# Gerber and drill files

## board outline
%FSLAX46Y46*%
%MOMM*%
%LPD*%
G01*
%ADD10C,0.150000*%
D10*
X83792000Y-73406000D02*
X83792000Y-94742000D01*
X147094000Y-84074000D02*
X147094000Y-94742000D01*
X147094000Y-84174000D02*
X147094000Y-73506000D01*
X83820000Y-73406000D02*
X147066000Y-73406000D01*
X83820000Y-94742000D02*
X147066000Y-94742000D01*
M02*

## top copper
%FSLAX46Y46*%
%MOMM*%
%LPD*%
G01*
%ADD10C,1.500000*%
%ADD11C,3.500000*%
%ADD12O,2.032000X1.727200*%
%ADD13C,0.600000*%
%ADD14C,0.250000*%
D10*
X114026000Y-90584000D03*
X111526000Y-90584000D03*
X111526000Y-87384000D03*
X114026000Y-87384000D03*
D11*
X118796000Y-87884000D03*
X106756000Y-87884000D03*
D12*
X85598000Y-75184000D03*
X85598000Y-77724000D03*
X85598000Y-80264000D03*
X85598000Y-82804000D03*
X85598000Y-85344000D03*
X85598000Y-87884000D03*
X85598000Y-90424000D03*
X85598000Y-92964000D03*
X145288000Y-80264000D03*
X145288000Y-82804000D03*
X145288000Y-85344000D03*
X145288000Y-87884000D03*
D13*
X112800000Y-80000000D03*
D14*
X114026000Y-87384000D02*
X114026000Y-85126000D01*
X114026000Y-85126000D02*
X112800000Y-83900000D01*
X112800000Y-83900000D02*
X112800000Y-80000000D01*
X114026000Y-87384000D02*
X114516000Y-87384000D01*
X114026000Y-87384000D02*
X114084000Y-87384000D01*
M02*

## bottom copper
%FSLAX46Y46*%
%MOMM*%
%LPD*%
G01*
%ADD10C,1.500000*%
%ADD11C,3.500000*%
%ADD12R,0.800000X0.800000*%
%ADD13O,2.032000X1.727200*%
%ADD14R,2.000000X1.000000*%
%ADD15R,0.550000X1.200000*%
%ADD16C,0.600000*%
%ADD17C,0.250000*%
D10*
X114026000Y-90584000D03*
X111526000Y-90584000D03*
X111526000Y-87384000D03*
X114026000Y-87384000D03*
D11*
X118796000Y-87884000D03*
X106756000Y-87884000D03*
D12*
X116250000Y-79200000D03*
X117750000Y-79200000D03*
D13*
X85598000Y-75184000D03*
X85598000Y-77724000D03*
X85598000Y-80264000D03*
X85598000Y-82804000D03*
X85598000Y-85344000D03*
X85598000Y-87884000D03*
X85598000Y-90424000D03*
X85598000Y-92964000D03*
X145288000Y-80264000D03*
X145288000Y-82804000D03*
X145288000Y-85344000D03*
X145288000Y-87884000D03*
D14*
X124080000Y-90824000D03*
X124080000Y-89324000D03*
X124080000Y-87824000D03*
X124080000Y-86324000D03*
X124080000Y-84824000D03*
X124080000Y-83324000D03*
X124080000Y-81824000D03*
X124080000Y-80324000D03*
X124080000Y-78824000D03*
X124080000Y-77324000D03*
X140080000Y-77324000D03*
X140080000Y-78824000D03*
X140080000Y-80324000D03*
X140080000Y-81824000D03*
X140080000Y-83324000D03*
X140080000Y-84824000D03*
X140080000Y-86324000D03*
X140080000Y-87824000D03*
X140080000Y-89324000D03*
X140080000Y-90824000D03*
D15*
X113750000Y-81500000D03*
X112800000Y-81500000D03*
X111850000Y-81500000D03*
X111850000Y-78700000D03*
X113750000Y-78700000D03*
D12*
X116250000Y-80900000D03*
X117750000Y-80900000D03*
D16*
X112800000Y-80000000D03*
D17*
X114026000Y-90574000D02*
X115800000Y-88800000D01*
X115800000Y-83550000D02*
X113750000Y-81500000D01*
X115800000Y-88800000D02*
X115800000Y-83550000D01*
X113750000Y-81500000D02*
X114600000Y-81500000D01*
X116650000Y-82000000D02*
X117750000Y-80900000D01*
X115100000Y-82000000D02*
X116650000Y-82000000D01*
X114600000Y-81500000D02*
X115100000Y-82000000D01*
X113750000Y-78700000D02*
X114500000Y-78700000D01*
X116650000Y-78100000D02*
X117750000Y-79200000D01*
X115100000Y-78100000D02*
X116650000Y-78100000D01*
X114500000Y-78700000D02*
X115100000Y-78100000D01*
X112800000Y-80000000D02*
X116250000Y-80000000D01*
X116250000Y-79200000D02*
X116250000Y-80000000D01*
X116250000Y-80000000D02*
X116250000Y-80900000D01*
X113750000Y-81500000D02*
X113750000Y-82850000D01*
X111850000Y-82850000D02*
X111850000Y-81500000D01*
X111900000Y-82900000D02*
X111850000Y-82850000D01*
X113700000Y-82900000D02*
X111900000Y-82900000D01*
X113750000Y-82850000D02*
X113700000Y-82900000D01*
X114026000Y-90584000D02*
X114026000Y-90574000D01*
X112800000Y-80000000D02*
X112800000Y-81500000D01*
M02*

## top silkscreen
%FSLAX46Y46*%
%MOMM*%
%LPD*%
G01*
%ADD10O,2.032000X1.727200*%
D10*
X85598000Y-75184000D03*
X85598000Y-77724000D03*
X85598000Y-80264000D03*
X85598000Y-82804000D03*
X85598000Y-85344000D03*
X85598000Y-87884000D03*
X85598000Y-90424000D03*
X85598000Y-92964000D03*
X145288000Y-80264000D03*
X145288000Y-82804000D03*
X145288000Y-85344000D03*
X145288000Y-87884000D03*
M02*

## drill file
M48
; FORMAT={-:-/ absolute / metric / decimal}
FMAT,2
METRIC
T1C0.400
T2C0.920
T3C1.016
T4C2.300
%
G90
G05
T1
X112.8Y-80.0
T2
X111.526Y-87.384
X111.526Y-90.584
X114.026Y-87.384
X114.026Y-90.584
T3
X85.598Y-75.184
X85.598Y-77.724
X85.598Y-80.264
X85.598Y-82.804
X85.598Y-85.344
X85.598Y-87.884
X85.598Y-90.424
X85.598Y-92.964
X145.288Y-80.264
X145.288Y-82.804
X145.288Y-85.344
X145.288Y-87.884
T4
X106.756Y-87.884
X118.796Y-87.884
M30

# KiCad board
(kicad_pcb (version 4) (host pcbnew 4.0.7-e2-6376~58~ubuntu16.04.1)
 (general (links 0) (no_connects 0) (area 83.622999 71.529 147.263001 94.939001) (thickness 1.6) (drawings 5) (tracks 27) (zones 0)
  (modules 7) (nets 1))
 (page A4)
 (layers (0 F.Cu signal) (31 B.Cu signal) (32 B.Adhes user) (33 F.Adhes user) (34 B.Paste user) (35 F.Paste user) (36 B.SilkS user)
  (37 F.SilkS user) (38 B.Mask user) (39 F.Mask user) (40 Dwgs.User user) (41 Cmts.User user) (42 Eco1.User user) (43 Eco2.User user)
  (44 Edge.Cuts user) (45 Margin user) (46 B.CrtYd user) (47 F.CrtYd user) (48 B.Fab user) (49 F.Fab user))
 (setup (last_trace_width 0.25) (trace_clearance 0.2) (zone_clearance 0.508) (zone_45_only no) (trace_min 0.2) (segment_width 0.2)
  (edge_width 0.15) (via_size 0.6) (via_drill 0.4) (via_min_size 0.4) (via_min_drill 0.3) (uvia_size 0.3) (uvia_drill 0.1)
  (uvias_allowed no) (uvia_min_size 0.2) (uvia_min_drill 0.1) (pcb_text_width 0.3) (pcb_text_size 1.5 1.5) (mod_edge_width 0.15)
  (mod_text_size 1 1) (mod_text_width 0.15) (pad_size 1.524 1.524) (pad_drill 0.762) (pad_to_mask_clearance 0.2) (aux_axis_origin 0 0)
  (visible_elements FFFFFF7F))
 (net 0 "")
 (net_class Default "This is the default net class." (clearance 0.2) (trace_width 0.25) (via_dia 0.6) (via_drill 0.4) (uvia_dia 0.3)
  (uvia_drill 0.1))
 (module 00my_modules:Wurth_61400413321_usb (layer B.Cu) (at 112.776 87.884)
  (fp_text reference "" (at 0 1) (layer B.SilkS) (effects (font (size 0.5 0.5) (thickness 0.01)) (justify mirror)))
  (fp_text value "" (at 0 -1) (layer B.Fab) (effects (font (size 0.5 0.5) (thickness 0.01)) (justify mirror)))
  (pad V thru_hole circle (at 1.25 2.7) (size 1.5 1.5) (drill 0.92) (layers *.Cu *.Mask B.SilkS))
  (pad - thru_hole circle (at -1.25 2.7) (size 1.5 1.5) (drill 0.92) (layers *.Cu *.Mask B.SilkS))
  (pad + thru_hole circle (at -1.25 -0.5) (size 1.5 1.5) (drill 0.92) (layers *.Cu *.Mask B.SilkS))
  (pad G thru_hole circle (at 1.25 -0.5) (size 1.5 1.5) (drill 0.92) (layers *.Cu *.Mask B.SilkS))
  (pad X thru_hole circle (at 6.02 0) (size 3.5 3.5) (drill 2.3) (layers *.Cu *.Mask B.SilkS))
  (pad X thru_hole circle (at -6.02 0) (size 3.5 3.5) (drill 2.3) (layers *.Cu *.Mask B.SilkS)))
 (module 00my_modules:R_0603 (layer B.Cu) (at 117 79.2)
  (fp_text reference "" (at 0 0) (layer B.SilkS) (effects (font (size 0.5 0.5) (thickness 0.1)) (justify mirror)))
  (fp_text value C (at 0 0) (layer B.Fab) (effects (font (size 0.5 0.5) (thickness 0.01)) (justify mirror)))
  (pad 1 smd rect (at -0.75 0) (size 0.8 0.8) (layers B.Cu B.Paste B.Mask))
  (pad 2 smd rect (at 0.75 0) (size 0.8 0.8) (layers B.Cu B.Paste B.Mask)))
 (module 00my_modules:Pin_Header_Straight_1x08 (layer F.Cu) (at 85.598 75.184)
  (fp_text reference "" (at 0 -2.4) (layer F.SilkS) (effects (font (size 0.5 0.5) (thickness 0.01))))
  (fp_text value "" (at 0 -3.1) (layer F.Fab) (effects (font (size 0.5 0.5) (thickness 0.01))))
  (pad 1 thru_hole oval (at 0 0) (size 2.032 1.7272) (drill 1.016) (layers *.Cu *.Mask F.SilkS))
  (pad 2 thru_hole oval (at 0 2.54) (size 2.032 1.7272) (drill 1.016) (layers *.Cu *.Mask F.SilkS))
  (pad 3 thru_hole oval (at 0 5.08) (size 2.032 1.7272) (drill 1.016) (layers *.Cu *.Mask F.SilkS))
  (pad 4 thru_hole oval (at 0 7.62) (size 2.032 1.7272) (drill 1.016) (layers *.Cu *.Mask F.SilkS))
  (pad 5 thru_hole oval (at 0 10.16) (size 2.032 1.7272) (drill 1.016) (layers *.Cu *.Mask F.SilkS))
  (pad 6 thru_hole oval (at 0 12.7) (size 2.032 1.7272) (drill 1.016) (layers *.Cu *.Mask F.SilkS))
  (pad 7 thru_hole oval (at 0 15.24) (size 2.032 1.7272) (drill 1.016) (layers *.Cu *.Mask F.SilkS))
  (pad 8 thru_hole oval (at 0 17.78) (size 2.032 1.7272) (drill 1.016) (layers *.Cu *.Mask F.SilkS)))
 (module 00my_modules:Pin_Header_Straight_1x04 (layer F.Cu) (at 145.288 80.264)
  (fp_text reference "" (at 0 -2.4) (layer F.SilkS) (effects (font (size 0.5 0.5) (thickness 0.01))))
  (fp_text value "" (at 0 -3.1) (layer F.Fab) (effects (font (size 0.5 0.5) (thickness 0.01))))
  (pad 1 thru_hole oval (at 0 0) (size 2.032 1.7272) (drill 1.016) (layers *.Cu *.Mask F.SilkS))
  (pad 2 thru_hole oval (at 0 2.54) (size 2.032 1.7272) (drill 1.016) (layers *.Cu *.Mask F.SilkS))
  (pad 3 thru_hole oval (at 0 5.08) (size 2.032 1.7272) (drill 1.016) (layers *.Cu *.Mask F.SilkS))
  (pad 4 thru_hole oval (at 0 7.62) (size 2.032 1.7272) (drill 1.016) (layers *.Cu *.Mask F.SilkS)))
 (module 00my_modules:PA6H (layer B.Cu) (at 132.08 84.074)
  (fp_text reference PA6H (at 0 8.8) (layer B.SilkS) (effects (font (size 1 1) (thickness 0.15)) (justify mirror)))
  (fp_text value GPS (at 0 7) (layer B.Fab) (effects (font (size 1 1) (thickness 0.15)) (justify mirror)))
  (pad VCC smd rect (at -8 6.75) (size 2 1) (layers B.Cu B.Paste B.Mask))
  (pad 2 smd rect (at -8 5.25) (size 2 1) (layers B.Cu B.Paste B.Mask))
  (pad GND smd rect (at -8 3.75) (size 2 1) (layers B.Cu B.Paste B.Mask))
  (pad 4 smd rect (at -8 2.25) (size 2 1) (layers B.Cu B.Paste B.Mask))
  (pad 5 smd rect (at -8 0.75) (size 2 1) (layers B.Cu B.Paste B.Mask))
  (pad 6 smd rect (at -8 -0.75) (size 2 1) (layers B.Cu B.Paste B.Mask))
  (pad 7 smd rect (at -8 -2.25) (size 2 1) (layers B.Cu B.Paste B.Mask))
  (pad 8 smd rect (at -8 -3.75) (size 2 1) (layers B.Cu B.Paste B.Mask))
  (pad TX smd rect (at -8 -5.25) (size 2 1) (layers B.Cu B.Paste B.Mask))
  (pad RX smd rect (at -8 -6.75) (size 2 1) (layers B.Cu B.Paste B.Mask))
  (pad 11 smd rect (at 8 -6.75) (size 2 1) (layers B.Cu B.Paste B.Mask))
  (pad 12 smd rect (at 8 -5.25) (size 2 1) (layers B.Cu B.Paste B.Mask))
  (pad 13 smd rect (at 8 -3.75) (size 2 1) (layers B.Cu B.Paste B.Mask))
  (pad 14 smd rect (at 8 -2.25) (size 2 1) (layers B.Cu B.Paste B.Mask))
  (pad 15 smd rect (at 8 -0.75) (size 2 1) (layers B.Cu B.Paste B.Mask))
  (pad 16 smd rect (at 8 0.75) (size 2 1) (layers B.Cu B.Paste B.Mask))
  (pad 17 smd rect (at 8 2.25) (size 2 1) (layers B.Cu B.Paste B.Mask))
  (pad 18 smd rect (at 8 3.75) (size 2 1) (layers B.Cu B.Paste B.Mask))
  (pad 19 smd rect (at 8 5.25) (size 2 1) (layers B.Cu B.Paste B.Mask))
  (pad 20 smd rect (at 8 6.75) (size 2 1) (layers B.Cu B.Paste B.Mask)))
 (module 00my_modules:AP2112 (layer B.Cu) (at 112.8 80.1 90)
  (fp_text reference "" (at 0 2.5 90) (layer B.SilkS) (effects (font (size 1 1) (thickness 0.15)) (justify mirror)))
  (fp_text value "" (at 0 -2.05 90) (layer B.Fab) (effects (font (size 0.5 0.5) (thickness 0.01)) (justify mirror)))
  (pad VIN smd rect (at -1.4 0.95 90) (size 1.2 0.55) (layers B.Cu B.Paste B.Mask))
  (pad GND smd rect (at -1.4 0 90) (size 1.2 0.55) (layers B.Cu B.Paste B.Mask))
  (pad EN smd rect (at -1.4 -0.95 90) (size 1.2 0.55) (layers B.Cu B.Paste B.Mask))
  (pad NC smd rect (at 1.4 -0.95 90) (size 1.2 0.55) (layers B.Cu B.Paste B.Mask))
  (pad VOUT smd rect (at 1.4 0.95 90) (size 1.2 0.55) (layers B.Cu B.Paste B.Mask)))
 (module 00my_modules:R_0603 (layer B.Cu) (at 117 80.9)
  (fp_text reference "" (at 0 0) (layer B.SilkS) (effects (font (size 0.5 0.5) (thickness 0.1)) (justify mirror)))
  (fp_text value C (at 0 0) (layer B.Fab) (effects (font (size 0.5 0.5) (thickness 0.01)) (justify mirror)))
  (pad 1 smd rect (at -0.75 0) (size 0.8 0.8) (layers B.Cu B.Paste B.Mask))
  (pad 2 smd rect (at 0.75 0) (size 0.8 0.8) (layers B.Cu B.Paste B.Mask)))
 (gr_line (start 83.792 73.406) (end 83.792 94.742) (angle 90) (layer Edge.Cuts) (width 0.15))
 (gr_line (start 147.094 84.074) (end 147.094 94.742) (angle 90) (layer Edge.Cuts) (width 0.15))
 (gr_line (start 147.094 84.174) (end 147.094 73.506) (angle 90) (layer Edge.Cuts) (width 0.15))
 (gr_line (start 83.82 73.406) (end 147.066 73.406) (angle 90) (layer Edge.Cuts) (width 0.15))
 (gr_line (start 83.82 94.742) (end 147.066 94.742) (angle 90) (layer Edge.Cuts) (width 0.15))
 (segment (start 114.026 90.574) (end 115.8 88.8) (width 0.25) (layer B.Cu) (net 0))
 (segment (start 115.8 83.55) (end 113.75 81.5) (width 0.25) (layer B.Cu) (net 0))
 (segment (start 115.8 88.8) (end 115.8 83.55) (width 0.25) (layer B.Cu) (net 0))
 (segment (start 114.026 87.384) (end 114.026 85.126) (width 0.25) (layer F.Cu) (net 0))
 (segment (start 114.026 85.126) (end 112.8 83.9) (width 0.25) (layer F.Cu) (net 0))
 (segment (start 112.8 83.9) (end 112.8 80) (width 0.25) (layer F.Cu) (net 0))
 (via (at 112.8 80) (size 0.6) (drill 0.4) (layers F.Cu B.Cu) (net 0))
 (segment (start 114.026 87.384) (end 114.516 87.384) (width 0.25) (layer F.Cu) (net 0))
 (segment (start 113.75 81.5) (end 114.6 81.5) (width 0.25) (layer B.Cu) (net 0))
 (segment (start 116.65 82) (end 117.75 80.9) (width 0.25) (layer B.Cu) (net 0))
 (segment (start 115.1 82) (end 116.65 82) (width 0.25) (layer B.Cu) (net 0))
 (segment (start 114.6 81.5) (end 115.1 82) (width 0.25) (layer B.Cu) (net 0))
 (segment (start 113.75 78.7) (end 114.5 78.7) (width 0.25) (layer B.Cu) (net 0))
 (segment (start 116.65 78.1) (end 117.75 79.2) (width 0.25) (layer B.Cu) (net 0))
 (segment (start 115.1 78.1) (end 116.65 78.1) (width 0.25) (layer B.Cu) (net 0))
 (segment (start 114.5 78.7) (end 115.1 78.1) (width 0.25) (layer B.Cu) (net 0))
 (segment (start 112.8 80) (end 116.25 80) (width 0.25) (layer B.Cu) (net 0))
 (segment (start 116.25 79.2) (end 116.25 80) (width 0.25) (layer B.Cu) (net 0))
 (segment (start 116.25 80) (end 116.25 80.9) (width 0.25) (layer B.Cu) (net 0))
 (segment (start 114.026 87.384) (end 114.084 87.384) (width 0.25) (layer F.Cu) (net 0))
 (segment (start 113.75 81.5) (end 113.75 82.85) (width 0.25) (layer B.Cu) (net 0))
 (segment (start 111.85 82.85) (end 111.85 81.5) (width 0.25) (layer B.Cu) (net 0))
 (segment (start 111.9 82.9) (end 111.85 82.85) (width 0.25) (layer B.Cu) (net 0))
 (segment (start 113.7 82.9) (end 111.9 82.9) (width 0.25) (layer B.Cu) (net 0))
 (segment (start 113.75 82.85) (end 113.7 82.9) (width 0.25) (layer B.Cu) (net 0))
 (segment (start 114.026 90.584) (end 114.026 90.574) (width 0.25) (layer B.Cu) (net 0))
 (segment (start 112.8 80) (end 112.8 81.5) (width 0.25) (layer B.Cu) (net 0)))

